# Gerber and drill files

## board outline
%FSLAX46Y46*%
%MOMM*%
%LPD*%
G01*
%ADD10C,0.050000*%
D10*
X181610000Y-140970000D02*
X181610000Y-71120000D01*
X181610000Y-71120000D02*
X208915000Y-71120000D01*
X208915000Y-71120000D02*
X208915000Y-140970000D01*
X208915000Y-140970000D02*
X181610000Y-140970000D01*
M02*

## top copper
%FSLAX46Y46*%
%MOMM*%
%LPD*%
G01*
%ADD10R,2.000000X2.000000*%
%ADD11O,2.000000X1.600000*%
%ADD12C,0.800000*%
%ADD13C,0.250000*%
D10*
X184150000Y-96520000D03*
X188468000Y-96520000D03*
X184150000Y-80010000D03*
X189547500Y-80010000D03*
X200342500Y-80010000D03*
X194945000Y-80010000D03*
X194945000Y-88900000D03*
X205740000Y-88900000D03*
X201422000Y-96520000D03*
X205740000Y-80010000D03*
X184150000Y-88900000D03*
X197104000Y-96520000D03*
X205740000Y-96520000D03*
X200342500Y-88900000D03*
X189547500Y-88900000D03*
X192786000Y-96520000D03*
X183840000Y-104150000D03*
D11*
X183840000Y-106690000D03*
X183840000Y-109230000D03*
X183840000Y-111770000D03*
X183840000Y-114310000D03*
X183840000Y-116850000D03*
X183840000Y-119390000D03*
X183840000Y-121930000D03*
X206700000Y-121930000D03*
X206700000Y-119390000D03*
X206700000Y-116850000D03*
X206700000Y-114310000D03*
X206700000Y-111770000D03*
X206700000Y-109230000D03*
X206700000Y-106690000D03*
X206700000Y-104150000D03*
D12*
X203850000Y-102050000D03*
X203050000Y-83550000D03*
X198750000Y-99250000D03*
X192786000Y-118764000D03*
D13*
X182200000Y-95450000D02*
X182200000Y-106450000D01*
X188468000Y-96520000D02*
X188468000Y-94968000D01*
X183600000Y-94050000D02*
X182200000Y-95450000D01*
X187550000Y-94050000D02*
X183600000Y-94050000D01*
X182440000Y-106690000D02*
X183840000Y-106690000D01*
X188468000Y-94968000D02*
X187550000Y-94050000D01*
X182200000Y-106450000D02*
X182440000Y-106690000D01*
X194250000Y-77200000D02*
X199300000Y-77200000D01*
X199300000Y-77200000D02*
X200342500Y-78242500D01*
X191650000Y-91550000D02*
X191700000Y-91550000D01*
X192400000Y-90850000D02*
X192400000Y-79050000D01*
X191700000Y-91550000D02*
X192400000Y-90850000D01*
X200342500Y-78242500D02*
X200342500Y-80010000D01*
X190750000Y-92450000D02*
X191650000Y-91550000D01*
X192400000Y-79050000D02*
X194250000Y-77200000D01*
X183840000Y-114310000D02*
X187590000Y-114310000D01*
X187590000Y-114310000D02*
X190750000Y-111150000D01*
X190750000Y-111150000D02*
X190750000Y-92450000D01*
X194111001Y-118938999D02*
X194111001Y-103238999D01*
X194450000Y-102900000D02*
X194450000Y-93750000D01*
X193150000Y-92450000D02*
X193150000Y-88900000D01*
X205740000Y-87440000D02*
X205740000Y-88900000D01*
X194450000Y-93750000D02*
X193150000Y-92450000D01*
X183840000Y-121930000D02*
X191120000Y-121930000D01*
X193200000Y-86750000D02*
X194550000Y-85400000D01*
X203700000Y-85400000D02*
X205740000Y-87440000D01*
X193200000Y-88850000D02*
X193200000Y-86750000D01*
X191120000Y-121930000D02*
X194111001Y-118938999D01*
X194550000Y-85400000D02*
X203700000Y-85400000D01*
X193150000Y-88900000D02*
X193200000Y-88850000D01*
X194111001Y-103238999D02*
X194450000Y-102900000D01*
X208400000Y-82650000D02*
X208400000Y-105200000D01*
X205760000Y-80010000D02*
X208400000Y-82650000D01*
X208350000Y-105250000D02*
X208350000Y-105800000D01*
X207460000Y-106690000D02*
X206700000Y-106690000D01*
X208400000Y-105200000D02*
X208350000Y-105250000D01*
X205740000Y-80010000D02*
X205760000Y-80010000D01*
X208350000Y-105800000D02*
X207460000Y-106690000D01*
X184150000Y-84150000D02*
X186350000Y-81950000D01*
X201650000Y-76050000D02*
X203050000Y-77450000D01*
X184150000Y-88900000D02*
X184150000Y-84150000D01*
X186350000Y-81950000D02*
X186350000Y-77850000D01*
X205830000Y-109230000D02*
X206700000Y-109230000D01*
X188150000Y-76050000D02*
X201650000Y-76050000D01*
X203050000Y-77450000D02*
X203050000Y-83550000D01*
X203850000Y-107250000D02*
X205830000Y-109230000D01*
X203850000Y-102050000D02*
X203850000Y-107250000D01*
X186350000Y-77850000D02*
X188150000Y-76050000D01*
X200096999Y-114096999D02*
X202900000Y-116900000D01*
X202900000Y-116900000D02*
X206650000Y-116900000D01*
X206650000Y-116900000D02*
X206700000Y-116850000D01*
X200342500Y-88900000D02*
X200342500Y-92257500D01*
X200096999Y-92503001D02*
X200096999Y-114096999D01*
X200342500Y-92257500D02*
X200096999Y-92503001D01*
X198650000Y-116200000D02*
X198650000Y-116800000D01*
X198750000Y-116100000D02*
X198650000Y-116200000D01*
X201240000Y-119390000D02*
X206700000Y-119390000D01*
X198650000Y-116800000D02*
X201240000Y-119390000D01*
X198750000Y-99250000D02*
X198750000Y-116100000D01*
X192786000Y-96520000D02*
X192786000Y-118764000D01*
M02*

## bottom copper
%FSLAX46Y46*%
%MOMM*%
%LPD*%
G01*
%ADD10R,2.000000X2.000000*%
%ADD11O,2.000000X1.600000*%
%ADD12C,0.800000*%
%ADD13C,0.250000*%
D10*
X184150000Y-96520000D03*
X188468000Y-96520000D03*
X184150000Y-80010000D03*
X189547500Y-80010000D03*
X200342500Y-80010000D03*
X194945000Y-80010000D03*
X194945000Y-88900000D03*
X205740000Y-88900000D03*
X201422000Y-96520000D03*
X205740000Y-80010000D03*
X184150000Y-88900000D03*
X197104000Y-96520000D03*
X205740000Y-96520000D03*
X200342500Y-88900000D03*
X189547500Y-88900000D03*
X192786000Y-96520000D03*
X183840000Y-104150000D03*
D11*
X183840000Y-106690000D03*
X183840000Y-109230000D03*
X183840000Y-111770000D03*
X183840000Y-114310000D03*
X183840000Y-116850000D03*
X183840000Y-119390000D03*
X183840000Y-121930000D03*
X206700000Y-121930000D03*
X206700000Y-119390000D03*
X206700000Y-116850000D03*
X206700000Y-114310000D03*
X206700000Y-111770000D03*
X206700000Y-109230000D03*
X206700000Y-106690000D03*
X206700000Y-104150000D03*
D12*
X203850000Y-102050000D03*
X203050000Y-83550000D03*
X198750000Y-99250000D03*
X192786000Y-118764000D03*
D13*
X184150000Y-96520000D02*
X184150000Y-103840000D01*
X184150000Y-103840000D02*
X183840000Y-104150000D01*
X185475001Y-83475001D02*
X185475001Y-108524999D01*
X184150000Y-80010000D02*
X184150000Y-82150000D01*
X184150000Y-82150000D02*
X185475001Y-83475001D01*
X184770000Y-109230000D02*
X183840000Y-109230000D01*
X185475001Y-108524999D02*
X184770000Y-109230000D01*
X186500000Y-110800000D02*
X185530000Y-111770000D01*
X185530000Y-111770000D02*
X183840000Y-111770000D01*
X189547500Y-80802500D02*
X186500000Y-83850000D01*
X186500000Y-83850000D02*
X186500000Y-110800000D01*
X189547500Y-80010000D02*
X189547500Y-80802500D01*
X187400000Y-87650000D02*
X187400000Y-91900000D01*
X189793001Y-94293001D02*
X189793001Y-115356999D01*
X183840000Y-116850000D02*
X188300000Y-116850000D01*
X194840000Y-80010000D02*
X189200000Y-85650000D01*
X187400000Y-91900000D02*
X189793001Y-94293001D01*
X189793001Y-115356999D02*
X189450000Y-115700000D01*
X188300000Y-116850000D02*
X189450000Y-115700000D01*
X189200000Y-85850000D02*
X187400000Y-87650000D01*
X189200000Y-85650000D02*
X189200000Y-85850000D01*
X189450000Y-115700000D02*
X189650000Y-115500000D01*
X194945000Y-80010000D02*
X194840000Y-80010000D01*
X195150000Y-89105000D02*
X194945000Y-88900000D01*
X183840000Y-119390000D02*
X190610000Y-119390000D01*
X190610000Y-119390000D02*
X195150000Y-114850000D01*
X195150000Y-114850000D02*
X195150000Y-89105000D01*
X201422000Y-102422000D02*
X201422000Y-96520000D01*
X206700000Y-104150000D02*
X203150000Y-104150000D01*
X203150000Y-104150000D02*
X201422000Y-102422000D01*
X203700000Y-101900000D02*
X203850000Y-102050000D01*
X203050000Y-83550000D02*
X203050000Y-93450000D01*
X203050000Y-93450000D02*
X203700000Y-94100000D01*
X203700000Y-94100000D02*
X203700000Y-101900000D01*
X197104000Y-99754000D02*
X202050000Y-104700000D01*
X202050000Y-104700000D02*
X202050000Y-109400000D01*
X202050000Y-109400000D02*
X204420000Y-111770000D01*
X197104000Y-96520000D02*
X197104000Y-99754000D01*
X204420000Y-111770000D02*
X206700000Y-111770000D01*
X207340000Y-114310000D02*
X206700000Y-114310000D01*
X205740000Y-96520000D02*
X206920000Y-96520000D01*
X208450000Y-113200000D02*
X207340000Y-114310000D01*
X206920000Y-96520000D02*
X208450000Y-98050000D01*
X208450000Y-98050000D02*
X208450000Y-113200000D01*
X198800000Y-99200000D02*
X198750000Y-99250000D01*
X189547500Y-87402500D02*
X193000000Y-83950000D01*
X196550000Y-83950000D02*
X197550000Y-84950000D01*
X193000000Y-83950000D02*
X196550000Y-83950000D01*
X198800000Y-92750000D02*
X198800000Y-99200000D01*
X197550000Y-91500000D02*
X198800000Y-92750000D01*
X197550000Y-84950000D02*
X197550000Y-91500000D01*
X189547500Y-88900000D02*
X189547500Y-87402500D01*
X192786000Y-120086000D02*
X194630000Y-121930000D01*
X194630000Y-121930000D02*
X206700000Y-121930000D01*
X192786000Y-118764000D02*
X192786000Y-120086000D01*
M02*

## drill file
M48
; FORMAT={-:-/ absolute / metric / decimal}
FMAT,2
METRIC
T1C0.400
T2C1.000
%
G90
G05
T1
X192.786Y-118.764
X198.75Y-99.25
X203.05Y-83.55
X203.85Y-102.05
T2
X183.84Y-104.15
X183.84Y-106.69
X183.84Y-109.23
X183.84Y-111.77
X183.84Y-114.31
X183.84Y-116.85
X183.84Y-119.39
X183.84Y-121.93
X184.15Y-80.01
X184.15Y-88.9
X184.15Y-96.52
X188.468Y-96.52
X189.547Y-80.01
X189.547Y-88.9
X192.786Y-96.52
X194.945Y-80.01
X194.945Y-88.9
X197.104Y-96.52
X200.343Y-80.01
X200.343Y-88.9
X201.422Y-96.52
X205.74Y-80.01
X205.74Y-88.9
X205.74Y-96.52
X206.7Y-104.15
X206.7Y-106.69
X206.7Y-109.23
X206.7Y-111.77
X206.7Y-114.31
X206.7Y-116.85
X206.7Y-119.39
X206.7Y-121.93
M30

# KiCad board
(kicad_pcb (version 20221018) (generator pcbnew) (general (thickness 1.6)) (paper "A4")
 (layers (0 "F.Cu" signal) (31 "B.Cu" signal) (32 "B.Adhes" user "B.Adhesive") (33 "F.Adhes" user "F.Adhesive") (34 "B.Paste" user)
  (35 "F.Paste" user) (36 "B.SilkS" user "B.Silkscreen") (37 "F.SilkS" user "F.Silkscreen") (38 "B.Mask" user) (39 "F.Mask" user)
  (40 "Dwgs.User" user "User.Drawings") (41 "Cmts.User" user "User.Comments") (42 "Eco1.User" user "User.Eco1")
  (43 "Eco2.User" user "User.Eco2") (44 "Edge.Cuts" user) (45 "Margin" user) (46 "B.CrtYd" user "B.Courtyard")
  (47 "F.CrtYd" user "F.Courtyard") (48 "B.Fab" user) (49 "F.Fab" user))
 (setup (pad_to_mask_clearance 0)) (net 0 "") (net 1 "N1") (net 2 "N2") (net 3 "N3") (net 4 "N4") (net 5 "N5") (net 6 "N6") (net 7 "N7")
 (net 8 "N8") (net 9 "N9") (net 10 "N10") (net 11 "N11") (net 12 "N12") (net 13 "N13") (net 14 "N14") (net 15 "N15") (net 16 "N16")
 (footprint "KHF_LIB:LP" (layer "F.Cu") (at 184.15 96.52)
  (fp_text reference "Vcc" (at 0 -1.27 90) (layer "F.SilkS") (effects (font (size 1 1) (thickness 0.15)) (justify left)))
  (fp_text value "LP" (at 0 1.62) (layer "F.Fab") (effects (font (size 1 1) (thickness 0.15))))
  (pad "1" thru_hole rect (at 0 0) (size 2 2) (drill 1) (layers "*.Cu" "*.Mask") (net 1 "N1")))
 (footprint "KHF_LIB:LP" (layer "F.Cu") (at 188.468 96.52)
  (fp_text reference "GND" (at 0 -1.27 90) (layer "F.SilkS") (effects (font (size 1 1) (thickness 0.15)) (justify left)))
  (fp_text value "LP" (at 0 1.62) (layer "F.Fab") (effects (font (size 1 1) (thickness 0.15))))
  (pad "1" thru_hole rect (at 0 0) (size 2 2) (drill 1) (layers "*.Cu" "*.Mask") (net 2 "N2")))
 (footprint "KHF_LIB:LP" (layer "F.Cu") (at 184.15 80.01)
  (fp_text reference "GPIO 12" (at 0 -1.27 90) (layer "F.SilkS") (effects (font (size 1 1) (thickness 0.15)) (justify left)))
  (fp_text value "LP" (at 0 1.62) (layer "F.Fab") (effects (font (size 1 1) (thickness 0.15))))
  (pad "1" thru_hole rect (at 0 0) (size 2 2) (drill 1) (layers "*.Cu" "*.Mask") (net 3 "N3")))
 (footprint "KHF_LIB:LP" (layer "F.Cu") (at 189.5475 80.01)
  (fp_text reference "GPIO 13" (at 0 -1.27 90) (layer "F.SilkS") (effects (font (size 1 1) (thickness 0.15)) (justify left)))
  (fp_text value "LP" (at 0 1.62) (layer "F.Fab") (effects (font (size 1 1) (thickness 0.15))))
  (pad "1" thru_hole rect (at 0 0) (size 2 2) (drill 1) (layers "*.Cu" "*.Mask") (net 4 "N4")))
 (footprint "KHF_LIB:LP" (layer "F.Cu") (at 200.3425 80.01)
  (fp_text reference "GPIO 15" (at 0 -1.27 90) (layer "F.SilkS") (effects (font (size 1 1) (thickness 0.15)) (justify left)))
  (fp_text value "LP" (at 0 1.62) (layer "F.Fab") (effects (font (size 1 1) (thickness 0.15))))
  (pad "1" thru_hole rect (at 0 0) (size 2 2) (drill 1) (layers "*.Cu" "*.Mask") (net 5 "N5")))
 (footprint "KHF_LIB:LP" (layer "F.Cu") (at 194.945 80.01)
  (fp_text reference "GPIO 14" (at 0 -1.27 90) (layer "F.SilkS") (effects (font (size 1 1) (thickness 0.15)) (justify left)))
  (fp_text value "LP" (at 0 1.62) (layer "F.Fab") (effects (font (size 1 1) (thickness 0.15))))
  (pad "1" thru_hole rect (at 0 0) (size 2 2) (drill 1) (layers "*.Cu" "*.Mask") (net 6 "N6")))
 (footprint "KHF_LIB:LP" (layer "F.Cu") (at 194.945 88.9)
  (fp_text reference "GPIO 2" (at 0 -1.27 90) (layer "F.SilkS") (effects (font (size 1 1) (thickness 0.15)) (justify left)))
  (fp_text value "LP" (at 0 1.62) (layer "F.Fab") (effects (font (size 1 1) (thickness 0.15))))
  (pad "1" thru_hole rect (at 0 0) (size 2 2) (drill 1) (layers "*.Cu" "*.Mask") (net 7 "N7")))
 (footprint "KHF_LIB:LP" (layer "F.Cu") (at 205.74 88.9)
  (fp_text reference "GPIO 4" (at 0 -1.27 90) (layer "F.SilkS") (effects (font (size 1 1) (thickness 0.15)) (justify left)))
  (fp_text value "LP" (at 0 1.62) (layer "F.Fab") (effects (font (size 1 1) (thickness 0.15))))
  (pad "1" thru_hole rect (at 0 0) (size 2 2) (drill 1) (layers "*.Cu" "*.Mask") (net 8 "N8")))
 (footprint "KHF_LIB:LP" (layer "F.Cu") (at 201.422 96.52)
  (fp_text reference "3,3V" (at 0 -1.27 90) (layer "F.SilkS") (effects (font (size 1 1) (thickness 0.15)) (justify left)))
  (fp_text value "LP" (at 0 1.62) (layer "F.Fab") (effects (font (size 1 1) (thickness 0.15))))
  (pad "1" thru_hole rect (at 0 0) (size 2 2) (drill 1) (layers "*.Cu" "*.Mask") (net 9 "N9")))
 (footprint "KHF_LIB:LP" (layer "F.Cu") (at 205.74 80.01)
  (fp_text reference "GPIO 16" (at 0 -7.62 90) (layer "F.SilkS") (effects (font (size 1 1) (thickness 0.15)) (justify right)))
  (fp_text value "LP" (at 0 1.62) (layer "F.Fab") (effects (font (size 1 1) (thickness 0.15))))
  (pad "1" thru_hole rect (at 0 0) (size 2 2) (drill 1) (layers "*.Cu" "*.Mask") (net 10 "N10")))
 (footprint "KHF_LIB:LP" (layer "F.Cu") (at 184.15 88.9)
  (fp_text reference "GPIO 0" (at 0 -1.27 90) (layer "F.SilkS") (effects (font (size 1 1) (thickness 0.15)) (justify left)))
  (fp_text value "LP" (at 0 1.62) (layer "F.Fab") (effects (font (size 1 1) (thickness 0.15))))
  (pad "1" thru_hole rect (at 0 0) (size 2 2) (drill 1) (layers "*.Cu" "*.Mask") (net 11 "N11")))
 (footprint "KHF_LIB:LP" (layer "F.Cu") (at 197.104 96.52)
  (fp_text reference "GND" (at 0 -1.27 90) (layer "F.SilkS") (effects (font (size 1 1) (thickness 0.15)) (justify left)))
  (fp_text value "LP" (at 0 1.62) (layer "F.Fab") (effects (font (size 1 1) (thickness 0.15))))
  (pad "1" thru_hole rect (at 0 0) (size 2 2) (drill 1) (layers "*.Cu" "*.Mask") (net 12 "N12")))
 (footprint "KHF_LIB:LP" (layer "F.Cu") (at 205.74 96.52)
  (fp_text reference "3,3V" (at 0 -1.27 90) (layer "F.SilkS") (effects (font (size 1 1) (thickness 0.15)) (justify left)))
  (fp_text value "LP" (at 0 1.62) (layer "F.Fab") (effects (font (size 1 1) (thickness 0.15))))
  (pad "1" thru_hole rect (at 0 0) (size 2 2) (drill 1) (layers "*.Cu" "*.Mask") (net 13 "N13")))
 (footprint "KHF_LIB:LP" (layer "F.Cu") (at 200.3425 88.9)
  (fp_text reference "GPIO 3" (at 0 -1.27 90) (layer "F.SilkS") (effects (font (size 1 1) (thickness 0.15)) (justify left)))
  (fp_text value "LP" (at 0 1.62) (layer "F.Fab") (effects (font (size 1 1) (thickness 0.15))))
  (pad "1" thru_hole rect (at 0 0) (size 2 2) (drill 1) (layers "*.Cu" "*.Mask") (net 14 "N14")))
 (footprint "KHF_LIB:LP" (layer "F.Cu") (at 189.5475 88.9)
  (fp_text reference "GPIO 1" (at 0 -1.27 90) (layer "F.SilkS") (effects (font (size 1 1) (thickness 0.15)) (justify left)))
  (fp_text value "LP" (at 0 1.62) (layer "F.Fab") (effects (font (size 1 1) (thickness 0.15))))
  (pad "1" thru_hole rect (at 0 0) (size 2 2) (drill 1) (layers "*.Cu" "*.Mask") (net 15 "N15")))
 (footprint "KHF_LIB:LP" (layer "F.Cu") (at 192.786 96.52)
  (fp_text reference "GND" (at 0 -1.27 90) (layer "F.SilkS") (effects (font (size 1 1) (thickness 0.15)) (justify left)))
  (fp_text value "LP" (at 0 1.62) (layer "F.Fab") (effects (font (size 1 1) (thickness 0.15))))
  (pad "1" thru_hole rect (at 0 0) (size 2 2) (drill 1) (layers "*.Cu" "*.Mask") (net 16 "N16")))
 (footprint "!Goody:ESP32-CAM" (layer "F.Cu") (at 195.27 118.16)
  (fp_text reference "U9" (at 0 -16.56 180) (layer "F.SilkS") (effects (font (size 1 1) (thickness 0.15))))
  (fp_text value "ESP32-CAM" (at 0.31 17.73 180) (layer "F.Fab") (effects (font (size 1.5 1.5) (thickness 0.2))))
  (pad "1" thru_hole rect (at -11.43 -14.01) (size 2 2) (drill 1) (layers "*.Cu" "*.Mask") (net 1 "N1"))
  (pad "2" thru_hole oval (at -11.43 -11.47) (size 2 1.6) (drill 1) (layers "*.Cu" "*.Mask") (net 2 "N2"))
  (pad "3" thru_hole oval (at -11.43 -8.93) (size 2 1.6) (drill 1) (layers "*.Cu" "*.Mask") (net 3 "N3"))
  (pad "4" thru_hole oval (at -11.43 -6.39) (size 2 1.6) (drill 1) (layers "*.Cu" "*.Mask") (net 4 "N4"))
  (pad "5" thru_hole oval (at -11.43 -3.85) (size 2 1.6) (drill 1) (layers "*.Cu" "*.Mask") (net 5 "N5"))
  (pad "6" thru_hole oval (at -11.43 -1.31) (size 2 1.6) (drill 1) (layers "*.Cu" "*.Mask") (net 6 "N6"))
  (pad "7" thru_hole oval (at -11.43 1.23) (size 2 1.6) (drill 1) (layers "*.Cu" "*.Mask") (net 7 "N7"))
  (pad "8" thru_hole oval (at -11.43 3.77) (size 2 1.6) (drill 1) (layers "*.Cu" "*.Mask") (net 8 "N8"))
  (pad "9" thru_hole oval (at 11.43 3.77) (size 2 1.6) (drill 1) (layers "*.Cu" "*.Mask") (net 16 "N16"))
  (pad "10" thru_hole oval (at 11.43 1.23) (size 2 1.6) (drill 1) (layers "*.Cu" "*.Mask") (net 15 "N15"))
  (pad "11" thru_hole oval (at 11.43 -1.31) (size 2 1.6) (drill 1) (layers "*.Cu" "*.Mask") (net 14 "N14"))
  (pad "12" thru_hole oval (at 11.43 -3.85) (size 2 1.6) (drill 1) (layers "*.Cu" "*.Mask") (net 13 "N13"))
  (pad "13" thru_hole oval (at 11.43 -6.39) (size 2 1.6) (drill 1) (layers "*.Cu" "*.Mask") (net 12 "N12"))
  (pad "14" thru_hole oval (at 11.43 -8.93) (size 2 1.6) (drill 1) (layers "*.Cu" "*.Mask") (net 11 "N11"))
  (pad "15" thru_hole oval (at 11.43 -11.47) (size 2 1.6) (drill 1) (layers "*.Cu" "*.Mask") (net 10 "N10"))
  (pad "16" thru_hole oval (at 11.43 -14.01) (size 2 1.6) (drill 1) (layers "*.Cu" "*.Mask") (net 9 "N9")))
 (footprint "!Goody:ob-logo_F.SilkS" (layer "F.Cu") (at 195.58 119.38)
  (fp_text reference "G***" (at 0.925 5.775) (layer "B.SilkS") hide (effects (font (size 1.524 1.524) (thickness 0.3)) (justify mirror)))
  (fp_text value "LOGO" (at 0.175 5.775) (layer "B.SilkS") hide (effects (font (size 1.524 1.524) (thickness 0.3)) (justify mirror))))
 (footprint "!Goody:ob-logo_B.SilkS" (layer "F.Cu") (at 201.93 135.89)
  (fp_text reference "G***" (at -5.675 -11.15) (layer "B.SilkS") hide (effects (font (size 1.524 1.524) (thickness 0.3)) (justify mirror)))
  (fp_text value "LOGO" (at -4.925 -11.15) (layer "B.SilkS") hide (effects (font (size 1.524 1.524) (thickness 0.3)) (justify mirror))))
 (gr_line (start 181.61 140.97) (end 181.61 71.12) (stroke (width 0.05) (type solid)) (layer "Edge.Cuts"))
 (gr_line (start 181.61 71.12) (end 208.915 71.12) (stroke (width 0.05) (type solid)) (layer "Edge.Cuts"))
 (gr_line (start 208.915 71.12) (end 208.915 140.97) (stroke (width 0.05) (type solid)) (layer "Edge.Cuts"))
 (gr_line (start 208.915 140.97) (end 181.61 140.97) (stroke (width 0.05) (type solid)) (layer "Edge.Cuts"))
 (segment (start 184.15 96.52) (end 184.15 103.84) (width 0.25) (layer "B.Cu") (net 1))
 (segment (start 184.15 103.84) (end 183.84 104.15) (width 0.25) (layer "B.Cu") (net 1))
 (segment (start 182.2 95.45) (end 182.2 106.45) (width 0.25) (layer "F.Cu") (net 2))
 (segment (start 188.468 96.52) (end 188.468 94.968) (width 0.25) (layer "F.Cu") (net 2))
 (segment (start 183.6 94.05) (end 182.2 95.45) (width 0.25) (layer "F.Cu") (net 2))
 (segment (start 187.55 94.05) (end 183.6 94.05) (width 0.25) (layer "F.Cu") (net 2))
 (segment (start 182.44 106.69) (end 183.84 106.69) (width 0.25) (layer "F.Cu") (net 2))
 (segment (start 188.468 94.968) (end 187.55 94.05) (width 0.25) (layer "F.Cu") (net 2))
 (segment (start 182.2 106.45) (end 182.44 106.69) (width 0.25) (layer "F.Cu") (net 2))
 (segment (start 185.475001 83.475001) (end 185.475001 108.524999) (width 0.25) (layer "B.Cu") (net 3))
 (segment (start 184.15 80.01) (end 184.15 82.15) (width 0.25) (layer "B.Cu") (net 3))
 (segment (start 184.15 82.15) (end 185.475001 83.475001) (width 0.25) (layer "B.Cu") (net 3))
 (segment (start 184.77 109.23) (end 183.84 109.23) (width 0.25) (layer "B.Cu") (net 3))
 (segment (start 185.475001 108.524999) (end 184.77 109.23) (width 0.25) (layer "B.Cu") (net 3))
 (segment (start 186.5 110.8) (end 185.53 111.77) (width 0.25) (layer "B.Cu") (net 4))
 (segment (start 185.53 111.77) (end 183.84 111.77) (width 0.25) (layer "B.Cu") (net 4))
 (segment (start 189.5475 80.8025) (end 186.5 83.85) (width 0.25) (layer "B.Cu") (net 4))
 (segment (start 186.5 83.85) (end 186.5 110.8) (width 0.25) (layer "B.Cu") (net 4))
 (segment (start 189.5475 80.01) (end 189.5475 80.8025) (width 0.25) (layer "B.Cu") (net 4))
 (segment (start 194.25 77.2) (end 199.3 77.2) (width 0.25) (layer "F.Cu") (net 5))
 (segment (start 199.3 77.2) (end 200.3425 78.2425) (width 0.25) (layer "F.Cu") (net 5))
 (segment (start 191.65 91.55) (end 191.7 91.55) (width 0.25) (layer "F.Cu") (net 5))
 (segment (start 192.4 90.85) (end 192.4 79.05) (width 0.25) (layer "F.Cu") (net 5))
 (segment (start 191.7 91.55) (end 192.4 90.85) (width 0.25) (layer "F.Cu") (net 5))
 (segment (start 200.3425 78.2425) (end 200.3425 80.01) (width 0.25) (layer "F.Cu") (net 5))
 (segment (start 190.75 92.45) (end 191.65 91.55) (width 0.25) (layer "F.Cu") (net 5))
 (segment (start 192.4 79.05) (end 194.25 77.2) (width 0.25) (layer "F.Cu") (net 5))
 (segment (start 183.84 114.31) (end 187.59 114.31) (width 0.25) (layer "F.Cu") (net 5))
 (segment (start 187.59 114.31) (end 190.75 111.15) (width 0.25) (layer "F.Cu") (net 5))
 (segment (start 190.75 111.15) (end 190.75 92.45) (width 0.25) (layer "F.Cu") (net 5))
 (segment (start 187.4 87.65) (end 187.4 91.9) (width 0.25) (layer "B.Cu") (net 6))
 (segment (start 189.793001 94.293001) (end 189.793001 115.356999) (width 0.25) (layer "B.Cu") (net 6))
 (segment (start 183.84 116.85) (end 188.3 116.85) (width 0.25) (layer "B.Cu") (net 6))
 (segment (start 194.84 80.01) (end 189.2 85.65) (width 0.25) (layer "B.Cu") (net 6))
 (segment (start 187.4 91.9) (end 189.793001 94.293001) (width 0.25) (layer "B.Cu") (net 6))
 (segment (start 189.793001 115.356999) (end 189.45 115.7) (width 0.25) (layer "B.Cu") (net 6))
 (segment (start 188.3 116.85) (end 189.45 115.7) (width 0.25) (layer "B.Cu") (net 6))
 (segment (start 189.2 85.85) (end 187.4 87.65) (width 0.25) (layer "B.Cu") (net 6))
 (segment (start 189.2 85.65) (end 189.2 85.85) (width 0.25) (layer "B.Cu") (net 6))
 (segment (start 189.45 115.7) (end 189.65 115.5) (width 0.25) (layer "B.Cu") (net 6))
 (segment (start 194.945 80.01) (end 194.84 80.01) (width 0.25) (layer "B.Cu") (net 6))
 (segment (start 195.15 89.105) (end 194.945 88.9) (width 0.25) (layer "B.Cu") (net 7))
 (segment (start 183.84 119.39) (end 190.61 119.39) (width 0.25) (layer "B.Cu") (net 7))
 (segment (start 190.61 119.39) (end 195.15 114.85) (width 0.25) (layer "B.Cu") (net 7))
 (segment (start 195.15 114.85) (end 195.15 89.105) (width 0.25) (layer "B.Cu") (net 7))
 (segment (start 194.111001 118.938999) (end 194.111001 103.238999) (width 0.25) (layer "F.Cu") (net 8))
 (segment (start 194.45 102.9) (end 194.45 93.75) (width 0.25) (layer "F.Cu") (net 8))
 (segment (start 193.15 92.45) (end 193.15 88.9) (width 0.25) (layer "F.Cu") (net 8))
 (segment (start 205.74 87.44) (end 205.74 88.9) (width 0.25) (layer "F.Cu") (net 8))
 (segment (start 194.45 93.75) (end 193.15 92.45) (width 0.25) (layer "F.Cu") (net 8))
 (segment (start 183.84 121.93) (end 191.12 121.93) (width 0.25) (layer "F.Cu") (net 8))
 (segment (start 193.2 86.75) (end 194.55 85.4) (width 0.25) (layer "F.Cu") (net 8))
 (segment (start 203.7 85.4) (end 205.74 87.44) (width 0.25) (layer "F.Cu") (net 8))
 (segment (start 193.2 88.85) (end 193.2 86.75) (width 0.25) (layer "F.Cu") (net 8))
 (segment (start 191.12 121.93) (end 194.111001 118.938999) (width 0.25) (layer "F.Cu") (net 8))
 (segment (start 194.55 85.4) (end 203.7 85.4) (width 0.25) (layer "F.Cu") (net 8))
 (segment (start 193.15 88.9) (end 193.2 88.85) (width 0.25) (layer "F.Cu") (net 8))
 (segment (start 194.111001 103.238999) (end 194.45 102.9) (width 0.25) (layer "F.Cu") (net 8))
 (segment (start 201.422 102.422) (end 201.422 96.52) (width 0.25) (layer "B.Cu") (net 9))
 (segment (start 206.7 104.15) (end 203.15 104.15) (width 0.25) (layer "B.Cu") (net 9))
 (segment (start 203.15 104.15) (end 201.422 102.422) (width 0.25) (layer "B.Cu") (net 9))
 (segment (start 208.4 82.65) (end 208.4 105.2) (width 0.25) (layer "F.Cu") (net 10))
 (segment (start 205.76 80.01) (end 208.4 82.65) (width 0.25) (layer "F.Cu") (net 10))
 (segment (start 208.35 105.25) (end 208.35 105.8) (width 0.25) (layer "F.Cu") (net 10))
 (segment (start 207.46 106.69) (end 206.7 106.69) (width 0.25) (layer "F.Cu") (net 10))
 (segment (start 208.4 105.2) (end 208.35 105.25) (width 0.25) (layer "F.Cu") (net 10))
 (segment (start 205.74 80.01) (end 205.76 80.01) (width 0.25) (layer "F.Cu") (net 10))
 (segment (start 208.35 105.8) (end 207.46 106.69) (width 0.25) (layer "F.Cu") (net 10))
 (segment (start 184.15 84.15) (end 186.35 81.95) (width 0.25) (layer "F.Cu") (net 11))
 (segment (start 201.65 76.05) (end 203.05 77.45) (width 0.25) (layer "F.Cu") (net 11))
 (segment (start 184.15 88.9) (end 184.15 84.15) (width 0.25) (layer "F.Cu") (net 11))
 (segment (start 186.35 81.95) (end 186.35 77.85) (width 0.25) (layer "F.Cu") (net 11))
 (segment (start 205.83 109.23) (end 206.7 109.23) (width 0.25) (layer "F.Cu") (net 11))
 (segment (start 188.15 76.05) (end 201.65 76.05) (width 0.25) (layer "F.Cu") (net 11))
 (segment (start 203.05 77.45) (end 203.05 83.55) (width 0.25) (layer "F.Cu") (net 11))
 (segment (start 203.85 107.25) (end 205.83 109.23) (width 0.25) (layer "F.Cu") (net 11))
 (segment (start 203.85 102.05) (end 203.85 107.25) (width 0.25) (layer "F.Cu") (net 11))
 (segment (start 186.35 77.85) (end 188.15 76.05) (width 0.25) (layer "F.Cu") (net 11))
 (via (at 203.85 102.05) (size 0.8) (drill 0.4) (layers "F.Cu" "B.Cu") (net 11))
 (via (at 203.05 83.55) (size 0.8) (drill 0.4) (layers "F.Cu" "B.Cu") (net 11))
 (segment (start 203.7 101.9) (end 203.85 102.05) (width 0.25) (layer "B.Cu") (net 11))
 (segment (start 203.05 83.55) (end 203.05 93.45) (width 0.25) (layer "B.Cu") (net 11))
 (segment (start 203.05 93.45) (end 203.7 94.1) (width 0.25) (layer "B.Cu") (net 11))
 (segment (start 203.7 94.1) (end 203.7 101.9) (width 0.25) (layer "B.Cu") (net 11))
 (segment (start 197.104 99.754) (end 202.05 104.7) (width 0.25) (layer "B.Cu") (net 12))
 (segment (start 202.05 104.7) (end 202.05 109.4) (width 0.25) (layer "B.Cu") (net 12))
 (segment (start 202.05 109.4) (end 204.42 111.77) (width 0.25) (layer "B.Cu") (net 12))
 (segment (start 197.104 96.52) (end 197.104 99.754) (width 0.25) (layer "B.Cu") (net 12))
 (segment (start 204.42 111.77) (end 206.7 111.77) (width 0.25) (layer "B.Cu") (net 12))
 (segment (start 207.34 114.31) (end 206.7 114.31) (width 0.25) (layer "B.Cu") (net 13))
 (segment (start 205.74 96.52) (end 206.92 96.52) (width 0.25) (layer "B.Cu") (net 13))
 (segment (start 208.45 113.2) (end 207.34 114.31) (width 0.25) (layer "B.Cu") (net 13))
 (segment (start 206.92 96.52) (end 208.45 98.05) (width 0.25) (layer "B.Cu") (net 13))
 (segment (start 208.45 98.05) (end 208.45 113.2) (width 0.25) (layer "B.Cu") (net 13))
 (segment (start 200.096999 114.096999) (end 202.9 116.9) (width 0.25) (layer "F.Cu") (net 14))
 (segment (start 202.9 116.9) (end 206.65 116.9) (width 0.25) (layer "F.Cu") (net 14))
 (segment (start 206.65 116.9) (end 206.7 116.85) (width 0.25) (layer "F.Cu") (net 14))
 (segment (start 200.3425 88.9) (end 200.3425 92.2575) (width 0.25) (layer "F.Cu") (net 14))
 (segment (start 200.096999 92.503001) (end 200.096999 114.096999) (width 0.25) (layer "F.Cu") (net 14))
 (segment (start 200.3425 92.2575) (end 200.096999 92.503001) (width 0.25) (layer "F.Cu") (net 14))
 (segment (start 198.65 116.2) (end 198.65 116.8) (width 0.25) (layer "F.Cu") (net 15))
 (segment (start 198.75 116.1) (end 198.65 116.2) (width 0.25) (layer "F.Cu") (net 15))
 (segment (start 201.24 119.39) (end 206.7 119.39) (width 0.25) (layer "F.Cu") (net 15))
 (segment (start 198.65 116.8) (end 201.24 119.39) (width 0.25) (layer "F.Cu") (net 15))
 (segment (start 198.75 99.25) (end 198.75 116.1) (width 0.25) (layer "F.Cu") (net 15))
 (via (at 198.75 99.25) (size 0.8) (drill 0.4) (layers "F.Cu" "B.Cu") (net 15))
 (segment (start 198.8 99.2) (end 198.75 99.25) (width 0.25) (layer "B.Cu") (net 15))
 (segment (start 189.5475 87.4025) (end 193 83.95) (width 0.25) (layer "B.Cu") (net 15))
 (segment (start 196.55 83.95) (end 197.55 84.95) (width 0.25) (layer "B.Cu") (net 15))
 (segment (start 193 83.95) (end 196.55 83.95) (width 0.25) (layer "B.Cu") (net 15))
 (segment (start 198.8 92.75) (end 198.8 99.2) (width 0.25) (layer "B.Cu") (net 15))
 (segment (start 197.55 91.5) (end 198.8 92.75) (width 0.25) (layer "B.Cu") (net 15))
 (segment (start 197.55 84.95) (end 197.55 91.5) (width 0.25) (layer "B.Cu") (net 15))
 (segment (start 189.5475 88.9) (end 189.5475 87.4025) (width 0.25) (layer "B.Cu") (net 15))
 (segment (start 192.786 96.52) (end 192.786 118.764) (width 0.25) (layer "F.Cu") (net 16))
 (via (at 192.786 118.764) (size 0.8) (drill 0.4) (layers "F.Cu" "B.Cu") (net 16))
 (segment (start 192.786 120.086) (end 194.63 121.93) (width 0.25) (layer "B.Cu") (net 16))
 (segment (start 194.63 121.93) (end 206.7 121.93) (width 0.25) (layer "B.Cu") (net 16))
 (segment (start 192.786 118.764) (end 192.786 120.086) (width 0.25) (layer "B.Cu") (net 16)))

